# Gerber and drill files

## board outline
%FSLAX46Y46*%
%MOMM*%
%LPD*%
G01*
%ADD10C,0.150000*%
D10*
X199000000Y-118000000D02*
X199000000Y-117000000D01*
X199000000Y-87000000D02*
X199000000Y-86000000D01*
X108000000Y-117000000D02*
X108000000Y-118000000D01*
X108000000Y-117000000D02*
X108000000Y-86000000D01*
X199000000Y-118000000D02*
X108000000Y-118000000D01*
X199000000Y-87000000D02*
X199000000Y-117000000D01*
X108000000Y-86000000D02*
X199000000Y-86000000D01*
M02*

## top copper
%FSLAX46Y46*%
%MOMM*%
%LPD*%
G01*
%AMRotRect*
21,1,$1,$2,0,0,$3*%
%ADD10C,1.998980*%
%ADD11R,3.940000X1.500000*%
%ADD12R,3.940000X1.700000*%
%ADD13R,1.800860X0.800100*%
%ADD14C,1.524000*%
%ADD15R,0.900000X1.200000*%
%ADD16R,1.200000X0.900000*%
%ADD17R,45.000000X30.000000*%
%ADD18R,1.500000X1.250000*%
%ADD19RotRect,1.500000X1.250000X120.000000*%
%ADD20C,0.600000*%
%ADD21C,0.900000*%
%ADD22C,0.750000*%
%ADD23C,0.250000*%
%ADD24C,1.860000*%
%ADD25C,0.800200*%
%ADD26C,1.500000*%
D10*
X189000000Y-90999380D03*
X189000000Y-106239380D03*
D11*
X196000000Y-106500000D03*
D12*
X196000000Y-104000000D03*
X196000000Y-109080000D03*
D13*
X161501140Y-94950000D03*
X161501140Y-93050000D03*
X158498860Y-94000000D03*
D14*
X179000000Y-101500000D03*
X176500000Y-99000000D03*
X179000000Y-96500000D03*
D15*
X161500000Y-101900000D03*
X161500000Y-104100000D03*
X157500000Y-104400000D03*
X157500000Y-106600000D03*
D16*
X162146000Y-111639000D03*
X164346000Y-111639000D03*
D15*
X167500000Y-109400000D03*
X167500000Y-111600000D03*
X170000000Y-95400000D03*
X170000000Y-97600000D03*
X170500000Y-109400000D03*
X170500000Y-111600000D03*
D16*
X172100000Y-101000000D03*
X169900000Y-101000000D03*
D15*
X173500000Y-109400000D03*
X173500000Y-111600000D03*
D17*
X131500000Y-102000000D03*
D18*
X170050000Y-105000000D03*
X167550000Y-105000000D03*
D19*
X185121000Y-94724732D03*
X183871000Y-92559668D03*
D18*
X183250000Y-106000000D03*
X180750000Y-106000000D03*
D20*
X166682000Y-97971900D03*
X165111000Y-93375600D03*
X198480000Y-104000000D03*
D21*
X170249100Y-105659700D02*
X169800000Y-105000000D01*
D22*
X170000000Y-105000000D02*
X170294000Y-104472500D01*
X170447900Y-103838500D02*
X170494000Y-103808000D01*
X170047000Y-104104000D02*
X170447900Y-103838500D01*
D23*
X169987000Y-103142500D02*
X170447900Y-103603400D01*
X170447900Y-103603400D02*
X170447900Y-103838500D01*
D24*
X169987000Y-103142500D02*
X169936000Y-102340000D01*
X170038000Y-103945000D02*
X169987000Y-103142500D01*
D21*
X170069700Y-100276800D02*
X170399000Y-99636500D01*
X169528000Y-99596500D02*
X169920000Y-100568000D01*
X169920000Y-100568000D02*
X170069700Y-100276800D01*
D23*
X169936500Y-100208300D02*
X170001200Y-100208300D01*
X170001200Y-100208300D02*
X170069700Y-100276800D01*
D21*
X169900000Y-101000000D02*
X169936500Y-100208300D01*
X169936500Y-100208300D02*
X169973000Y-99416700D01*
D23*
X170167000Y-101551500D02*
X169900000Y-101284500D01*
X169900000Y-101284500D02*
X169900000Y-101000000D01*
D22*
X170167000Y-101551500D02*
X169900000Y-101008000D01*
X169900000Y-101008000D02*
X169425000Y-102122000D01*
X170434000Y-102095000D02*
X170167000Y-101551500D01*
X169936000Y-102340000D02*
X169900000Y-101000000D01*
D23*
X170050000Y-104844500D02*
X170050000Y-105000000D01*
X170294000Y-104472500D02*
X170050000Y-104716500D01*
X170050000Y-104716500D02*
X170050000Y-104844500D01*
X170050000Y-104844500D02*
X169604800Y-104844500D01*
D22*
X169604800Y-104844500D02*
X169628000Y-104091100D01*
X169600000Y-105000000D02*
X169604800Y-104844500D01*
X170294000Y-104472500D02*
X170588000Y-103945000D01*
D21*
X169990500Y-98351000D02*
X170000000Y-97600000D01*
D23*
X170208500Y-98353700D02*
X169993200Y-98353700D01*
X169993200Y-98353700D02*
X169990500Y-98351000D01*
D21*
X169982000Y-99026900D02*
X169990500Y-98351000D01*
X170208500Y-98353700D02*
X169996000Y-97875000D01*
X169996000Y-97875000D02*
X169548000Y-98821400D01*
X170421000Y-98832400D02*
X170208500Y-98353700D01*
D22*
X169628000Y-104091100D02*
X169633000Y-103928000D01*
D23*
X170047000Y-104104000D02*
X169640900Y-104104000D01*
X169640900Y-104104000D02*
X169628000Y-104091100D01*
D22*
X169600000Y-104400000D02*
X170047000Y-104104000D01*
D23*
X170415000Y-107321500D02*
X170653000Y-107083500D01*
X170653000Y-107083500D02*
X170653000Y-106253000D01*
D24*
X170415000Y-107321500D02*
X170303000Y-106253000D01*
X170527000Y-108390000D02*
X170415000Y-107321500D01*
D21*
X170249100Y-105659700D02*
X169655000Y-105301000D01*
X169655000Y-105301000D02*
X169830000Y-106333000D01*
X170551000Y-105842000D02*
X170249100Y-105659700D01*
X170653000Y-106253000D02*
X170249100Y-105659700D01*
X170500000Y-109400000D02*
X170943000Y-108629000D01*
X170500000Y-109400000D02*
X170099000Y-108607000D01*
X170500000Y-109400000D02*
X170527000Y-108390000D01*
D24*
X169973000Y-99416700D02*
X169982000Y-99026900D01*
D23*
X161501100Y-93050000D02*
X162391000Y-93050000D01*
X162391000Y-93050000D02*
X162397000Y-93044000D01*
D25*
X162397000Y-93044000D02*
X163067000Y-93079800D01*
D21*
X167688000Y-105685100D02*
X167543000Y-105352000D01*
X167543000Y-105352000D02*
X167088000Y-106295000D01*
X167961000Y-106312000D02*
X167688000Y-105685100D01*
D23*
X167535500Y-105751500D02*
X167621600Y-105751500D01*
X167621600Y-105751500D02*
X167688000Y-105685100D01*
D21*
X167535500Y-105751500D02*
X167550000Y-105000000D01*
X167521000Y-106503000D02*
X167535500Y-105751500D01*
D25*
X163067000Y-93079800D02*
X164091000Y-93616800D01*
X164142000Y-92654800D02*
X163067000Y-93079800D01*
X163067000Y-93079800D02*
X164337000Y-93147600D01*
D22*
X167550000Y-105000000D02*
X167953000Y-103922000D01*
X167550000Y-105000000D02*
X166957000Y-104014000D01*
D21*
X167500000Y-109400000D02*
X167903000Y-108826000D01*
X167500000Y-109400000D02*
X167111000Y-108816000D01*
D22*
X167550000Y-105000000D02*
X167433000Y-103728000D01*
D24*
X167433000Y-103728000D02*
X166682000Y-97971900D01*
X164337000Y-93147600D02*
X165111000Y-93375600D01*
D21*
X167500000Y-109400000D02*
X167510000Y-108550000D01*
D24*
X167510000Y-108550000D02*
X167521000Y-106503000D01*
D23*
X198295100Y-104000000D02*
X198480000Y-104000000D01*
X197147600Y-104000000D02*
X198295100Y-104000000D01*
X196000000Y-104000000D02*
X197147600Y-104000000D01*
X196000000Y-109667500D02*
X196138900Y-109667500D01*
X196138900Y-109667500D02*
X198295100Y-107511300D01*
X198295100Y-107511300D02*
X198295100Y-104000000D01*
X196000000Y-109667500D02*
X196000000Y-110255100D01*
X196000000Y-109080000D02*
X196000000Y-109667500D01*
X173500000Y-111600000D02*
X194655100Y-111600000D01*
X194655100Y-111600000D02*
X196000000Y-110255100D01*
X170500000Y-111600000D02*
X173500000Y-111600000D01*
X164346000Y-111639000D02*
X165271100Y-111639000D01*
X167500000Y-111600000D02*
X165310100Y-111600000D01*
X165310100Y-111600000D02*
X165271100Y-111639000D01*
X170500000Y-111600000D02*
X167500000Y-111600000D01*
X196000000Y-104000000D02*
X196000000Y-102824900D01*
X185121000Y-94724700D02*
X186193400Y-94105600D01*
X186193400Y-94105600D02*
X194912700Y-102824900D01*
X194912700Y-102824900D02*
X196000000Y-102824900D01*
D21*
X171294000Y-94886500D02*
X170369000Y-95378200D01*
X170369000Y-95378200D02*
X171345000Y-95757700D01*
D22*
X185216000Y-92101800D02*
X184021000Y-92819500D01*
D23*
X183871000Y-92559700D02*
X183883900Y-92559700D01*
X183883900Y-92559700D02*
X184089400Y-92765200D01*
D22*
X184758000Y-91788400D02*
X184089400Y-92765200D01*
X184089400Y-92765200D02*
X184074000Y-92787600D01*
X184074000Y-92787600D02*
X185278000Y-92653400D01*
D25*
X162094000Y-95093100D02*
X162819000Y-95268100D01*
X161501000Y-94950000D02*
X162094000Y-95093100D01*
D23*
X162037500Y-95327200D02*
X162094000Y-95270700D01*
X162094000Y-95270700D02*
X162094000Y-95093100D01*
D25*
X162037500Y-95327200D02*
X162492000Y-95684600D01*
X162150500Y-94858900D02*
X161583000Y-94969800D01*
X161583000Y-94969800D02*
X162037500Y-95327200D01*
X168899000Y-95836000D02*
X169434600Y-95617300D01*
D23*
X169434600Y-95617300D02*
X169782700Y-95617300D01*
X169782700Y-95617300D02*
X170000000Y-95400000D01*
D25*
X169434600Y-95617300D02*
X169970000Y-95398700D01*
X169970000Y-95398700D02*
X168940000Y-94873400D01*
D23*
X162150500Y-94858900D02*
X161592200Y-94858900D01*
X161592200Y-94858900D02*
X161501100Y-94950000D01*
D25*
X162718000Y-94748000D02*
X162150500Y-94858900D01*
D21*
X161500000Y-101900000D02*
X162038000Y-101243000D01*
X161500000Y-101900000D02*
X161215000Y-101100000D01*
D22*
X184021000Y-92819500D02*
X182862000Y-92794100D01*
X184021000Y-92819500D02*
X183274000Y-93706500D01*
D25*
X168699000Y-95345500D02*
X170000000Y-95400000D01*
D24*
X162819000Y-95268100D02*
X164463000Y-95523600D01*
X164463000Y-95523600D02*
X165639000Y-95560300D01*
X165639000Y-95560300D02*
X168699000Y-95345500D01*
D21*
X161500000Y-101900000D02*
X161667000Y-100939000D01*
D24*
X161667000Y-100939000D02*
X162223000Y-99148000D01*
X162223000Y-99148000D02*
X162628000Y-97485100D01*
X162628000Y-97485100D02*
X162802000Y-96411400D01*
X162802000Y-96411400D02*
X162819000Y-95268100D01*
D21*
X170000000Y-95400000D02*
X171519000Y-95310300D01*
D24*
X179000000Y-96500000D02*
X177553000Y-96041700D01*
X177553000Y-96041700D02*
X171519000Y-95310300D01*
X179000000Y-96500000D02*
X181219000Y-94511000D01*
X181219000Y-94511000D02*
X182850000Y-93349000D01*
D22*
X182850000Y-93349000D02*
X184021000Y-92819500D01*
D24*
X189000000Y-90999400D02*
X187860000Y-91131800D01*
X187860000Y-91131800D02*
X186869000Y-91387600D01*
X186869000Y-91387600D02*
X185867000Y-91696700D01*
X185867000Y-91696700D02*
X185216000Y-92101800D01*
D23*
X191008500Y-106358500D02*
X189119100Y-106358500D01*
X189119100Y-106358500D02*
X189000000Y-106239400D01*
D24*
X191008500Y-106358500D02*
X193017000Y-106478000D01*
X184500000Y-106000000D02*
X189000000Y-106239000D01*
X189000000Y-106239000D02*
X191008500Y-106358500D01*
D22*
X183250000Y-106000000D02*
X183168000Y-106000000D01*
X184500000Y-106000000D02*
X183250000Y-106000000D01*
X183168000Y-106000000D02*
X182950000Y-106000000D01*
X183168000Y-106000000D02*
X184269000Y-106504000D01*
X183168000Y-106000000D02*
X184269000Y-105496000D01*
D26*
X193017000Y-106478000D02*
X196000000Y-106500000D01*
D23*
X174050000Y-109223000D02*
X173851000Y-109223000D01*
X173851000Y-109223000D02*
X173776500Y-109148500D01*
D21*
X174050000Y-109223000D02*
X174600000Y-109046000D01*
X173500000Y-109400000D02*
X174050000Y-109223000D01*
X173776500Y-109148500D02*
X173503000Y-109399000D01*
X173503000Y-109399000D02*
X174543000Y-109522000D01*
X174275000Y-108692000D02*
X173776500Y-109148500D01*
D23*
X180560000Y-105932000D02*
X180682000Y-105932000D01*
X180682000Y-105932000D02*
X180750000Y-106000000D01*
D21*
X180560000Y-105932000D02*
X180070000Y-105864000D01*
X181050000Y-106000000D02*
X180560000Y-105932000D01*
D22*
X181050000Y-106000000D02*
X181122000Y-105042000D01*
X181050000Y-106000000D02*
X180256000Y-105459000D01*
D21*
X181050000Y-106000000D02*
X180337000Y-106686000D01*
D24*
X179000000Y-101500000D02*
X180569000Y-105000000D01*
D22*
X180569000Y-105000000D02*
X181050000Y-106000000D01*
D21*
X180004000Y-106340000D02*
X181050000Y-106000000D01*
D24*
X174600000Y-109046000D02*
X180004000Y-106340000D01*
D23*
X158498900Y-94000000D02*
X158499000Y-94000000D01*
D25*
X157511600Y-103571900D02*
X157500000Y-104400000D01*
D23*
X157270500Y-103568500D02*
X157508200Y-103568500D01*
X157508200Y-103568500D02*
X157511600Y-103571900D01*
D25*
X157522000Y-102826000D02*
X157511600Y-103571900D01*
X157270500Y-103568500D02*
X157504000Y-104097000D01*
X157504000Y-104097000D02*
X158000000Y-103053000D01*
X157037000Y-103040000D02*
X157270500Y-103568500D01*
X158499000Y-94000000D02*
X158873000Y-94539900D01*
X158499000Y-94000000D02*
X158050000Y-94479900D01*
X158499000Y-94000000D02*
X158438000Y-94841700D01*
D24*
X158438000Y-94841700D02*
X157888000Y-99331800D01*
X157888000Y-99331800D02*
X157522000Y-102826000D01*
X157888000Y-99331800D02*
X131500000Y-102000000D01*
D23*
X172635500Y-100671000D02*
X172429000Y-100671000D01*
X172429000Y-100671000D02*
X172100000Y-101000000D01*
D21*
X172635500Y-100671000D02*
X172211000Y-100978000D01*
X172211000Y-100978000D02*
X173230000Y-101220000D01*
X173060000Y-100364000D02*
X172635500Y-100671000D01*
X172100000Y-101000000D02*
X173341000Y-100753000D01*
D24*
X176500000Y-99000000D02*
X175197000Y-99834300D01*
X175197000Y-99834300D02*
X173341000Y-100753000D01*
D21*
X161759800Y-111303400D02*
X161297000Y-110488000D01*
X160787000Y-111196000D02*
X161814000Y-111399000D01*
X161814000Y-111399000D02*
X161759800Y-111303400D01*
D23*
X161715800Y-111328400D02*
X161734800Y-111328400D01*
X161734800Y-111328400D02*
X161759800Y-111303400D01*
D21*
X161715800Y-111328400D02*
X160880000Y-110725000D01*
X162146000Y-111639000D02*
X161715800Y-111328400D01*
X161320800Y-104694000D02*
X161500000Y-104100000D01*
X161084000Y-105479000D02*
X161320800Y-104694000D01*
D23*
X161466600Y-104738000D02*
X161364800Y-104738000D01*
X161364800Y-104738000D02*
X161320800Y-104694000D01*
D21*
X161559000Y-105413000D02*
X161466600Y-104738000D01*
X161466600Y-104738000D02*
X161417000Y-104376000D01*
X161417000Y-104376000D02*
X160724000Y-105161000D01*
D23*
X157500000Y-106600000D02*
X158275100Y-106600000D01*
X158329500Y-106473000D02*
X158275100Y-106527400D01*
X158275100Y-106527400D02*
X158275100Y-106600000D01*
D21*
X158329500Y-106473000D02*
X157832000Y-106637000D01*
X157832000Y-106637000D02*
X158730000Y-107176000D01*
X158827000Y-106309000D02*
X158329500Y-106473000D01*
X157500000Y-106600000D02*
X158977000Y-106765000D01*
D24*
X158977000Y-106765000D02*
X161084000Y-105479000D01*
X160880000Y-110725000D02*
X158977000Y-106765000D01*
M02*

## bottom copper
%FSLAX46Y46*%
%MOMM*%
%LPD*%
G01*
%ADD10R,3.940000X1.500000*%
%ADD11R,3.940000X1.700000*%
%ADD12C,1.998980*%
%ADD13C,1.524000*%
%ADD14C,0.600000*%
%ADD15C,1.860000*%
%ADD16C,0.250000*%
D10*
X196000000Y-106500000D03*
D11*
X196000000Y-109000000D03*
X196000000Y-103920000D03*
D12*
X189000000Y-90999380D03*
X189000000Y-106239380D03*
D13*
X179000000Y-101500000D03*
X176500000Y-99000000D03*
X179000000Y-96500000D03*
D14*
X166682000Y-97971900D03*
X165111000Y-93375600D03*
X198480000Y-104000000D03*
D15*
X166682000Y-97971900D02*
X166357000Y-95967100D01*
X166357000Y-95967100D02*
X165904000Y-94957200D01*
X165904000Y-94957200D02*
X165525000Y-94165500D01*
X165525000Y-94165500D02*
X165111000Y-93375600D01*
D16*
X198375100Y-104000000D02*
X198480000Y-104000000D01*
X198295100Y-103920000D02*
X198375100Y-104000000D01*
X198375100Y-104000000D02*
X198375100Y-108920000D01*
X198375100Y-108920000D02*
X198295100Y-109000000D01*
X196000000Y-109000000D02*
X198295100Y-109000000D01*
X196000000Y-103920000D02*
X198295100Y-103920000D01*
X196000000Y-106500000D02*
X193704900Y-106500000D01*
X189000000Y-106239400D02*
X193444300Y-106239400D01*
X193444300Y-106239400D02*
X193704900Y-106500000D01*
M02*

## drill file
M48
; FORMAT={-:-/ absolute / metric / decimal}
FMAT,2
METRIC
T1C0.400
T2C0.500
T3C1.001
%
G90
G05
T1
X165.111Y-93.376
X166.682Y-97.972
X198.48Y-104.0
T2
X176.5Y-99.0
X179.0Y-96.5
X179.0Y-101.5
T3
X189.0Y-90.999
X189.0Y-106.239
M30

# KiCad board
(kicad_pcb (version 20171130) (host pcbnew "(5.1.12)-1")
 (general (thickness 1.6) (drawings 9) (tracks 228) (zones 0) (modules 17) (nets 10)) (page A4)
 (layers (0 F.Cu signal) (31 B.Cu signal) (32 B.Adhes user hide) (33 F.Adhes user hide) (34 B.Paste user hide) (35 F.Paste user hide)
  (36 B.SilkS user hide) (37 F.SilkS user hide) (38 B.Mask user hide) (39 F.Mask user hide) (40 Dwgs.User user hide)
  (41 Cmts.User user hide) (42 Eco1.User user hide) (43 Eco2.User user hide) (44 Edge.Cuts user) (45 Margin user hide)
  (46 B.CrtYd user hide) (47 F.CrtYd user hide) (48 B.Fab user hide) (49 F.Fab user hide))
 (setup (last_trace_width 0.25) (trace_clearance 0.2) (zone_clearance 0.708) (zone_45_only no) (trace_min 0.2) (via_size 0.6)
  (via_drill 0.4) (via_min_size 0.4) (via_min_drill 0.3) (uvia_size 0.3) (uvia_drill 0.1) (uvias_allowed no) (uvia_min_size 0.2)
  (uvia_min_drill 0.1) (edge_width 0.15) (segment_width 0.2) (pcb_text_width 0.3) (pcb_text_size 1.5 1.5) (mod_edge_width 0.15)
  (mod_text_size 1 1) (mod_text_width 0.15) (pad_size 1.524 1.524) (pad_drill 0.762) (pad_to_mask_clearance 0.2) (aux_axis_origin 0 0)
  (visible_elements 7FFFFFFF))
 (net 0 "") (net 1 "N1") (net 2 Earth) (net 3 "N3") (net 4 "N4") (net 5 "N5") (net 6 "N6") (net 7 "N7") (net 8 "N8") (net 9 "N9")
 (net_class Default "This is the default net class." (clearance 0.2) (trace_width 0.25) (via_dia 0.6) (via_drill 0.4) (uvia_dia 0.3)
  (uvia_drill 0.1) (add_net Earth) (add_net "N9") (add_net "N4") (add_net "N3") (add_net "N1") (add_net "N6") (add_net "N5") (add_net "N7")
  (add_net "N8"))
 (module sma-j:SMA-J (layer B.Cu) (at 196 109)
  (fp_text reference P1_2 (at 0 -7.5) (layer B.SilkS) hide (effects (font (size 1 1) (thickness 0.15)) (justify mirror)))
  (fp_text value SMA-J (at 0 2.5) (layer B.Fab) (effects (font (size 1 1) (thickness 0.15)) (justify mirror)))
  (pad 1 smd rect (at 0 -2.5) (size 3.94 1.5) (layers B.Cu B.Paste B.Mask) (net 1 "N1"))
  (pad 2 smd rect (at 0 0) (size 3.94 1.7) (layers B.Cu B.Paste B.Mask) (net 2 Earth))
  (pad 2 smd rect (at 0 -5.08) (size 3.94 1.7) (layers B.Cu B.Paste B.Mask) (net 2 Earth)))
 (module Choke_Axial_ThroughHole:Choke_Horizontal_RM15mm (layer F.Cu) (at 189 98.5 270)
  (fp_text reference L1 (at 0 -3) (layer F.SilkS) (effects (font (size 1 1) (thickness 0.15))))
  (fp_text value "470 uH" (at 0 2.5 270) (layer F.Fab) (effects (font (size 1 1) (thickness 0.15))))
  (pad 1 thru_hole circle (at -7.50062 0 270) (size 1.99898 1.99898) (drill 1.00076) (layers *.Cu *.Mask F.SilkS) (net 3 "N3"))
  (pad 2 thru_hole circle (at 7.73938 0 270) (size 1.99898 1.99898) (drill 1.00076) (layers *.Cu *.Mask F.SilkS) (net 1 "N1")))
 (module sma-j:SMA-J (layer F.Cu) (at 196 104)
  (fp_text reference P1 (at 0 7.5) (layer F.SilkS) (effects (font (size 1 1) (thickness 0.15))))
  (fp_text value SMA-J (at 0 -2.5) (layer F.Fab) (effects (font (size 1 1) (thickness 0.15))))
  (pad 1 smd rect (at 0 2.5) (size 3.94 1.5) (layers F.Cu F.Paste F.Mask) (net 1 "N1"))
  (pad 2 smd rect (at 0 0) (size 3.94 1.7) (layers F.Cu F.Paste F.Mask) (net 2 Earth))
  (pad 2 smd rect (at 0 5.08) (size 3.94 1.7) (layers F.Cu F.Paste F.Mask) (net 2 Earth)))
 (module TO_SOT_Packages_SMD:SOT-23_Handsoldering (layer F.Cu) (at 160 94 90)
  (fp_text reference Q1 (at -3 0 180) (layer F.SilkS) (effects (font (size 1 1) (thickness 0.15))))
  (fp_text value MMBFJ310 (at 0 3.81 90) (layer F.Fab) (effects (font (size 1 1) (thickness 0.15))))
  (pad 1 smd rect (at -0.95 1.50114 90) (size 0.8001 1.80086) (layers F.Cu F.Paste F.Mask) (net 3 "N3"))
  (pad 2 smd rect (at 0.95 1.50114 90) (size 0.8001 1.80086) (layers F.Cu F.Paste F.Mask) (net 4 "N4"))
  (pad 3 smd rect (at 0 -1.50114 90) (size 0.8001 1.80086) (layers F.Cu F.Paste F.Mask) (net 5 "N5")))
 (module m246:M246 (layer F.Cu) (at 179 99 270)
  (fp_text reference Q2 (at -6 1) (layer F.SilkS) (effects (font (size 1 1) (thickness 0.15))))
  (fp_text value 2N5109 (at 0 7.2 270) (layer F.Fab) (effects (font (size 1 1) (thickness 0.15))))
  (pad 1 thru_hole circle (at 2.5 0 270) (size 1.524 1.524) (drill 0.5) (layers *.Cu *.Mask F.SilkS) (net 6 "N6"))
  (pad 2 thru_hole circle (at 0 2.5 270) (size 1.524 1.524) (drill 0.5) (layers *.Cu *.Mask F.SilkS) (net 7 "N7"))
  (pad 3 thru_hole circle (at -2.5 0 270) (size 1.524 1.524) (drill 0.5) (layers *.Cu *.Mask F.SilkS) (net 3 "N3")))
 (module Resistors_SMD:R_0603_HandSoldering (layer F.Cu) (at 161.5 103 270)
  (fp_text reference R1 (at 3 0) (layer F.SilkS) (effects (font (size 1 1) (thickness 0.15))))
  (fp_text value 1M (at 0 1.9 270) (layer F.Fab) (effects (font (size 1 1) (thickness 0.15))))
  (pad 1 smd rect (at -1.1 0 270) (size 1.2 0.9) (layers F.Cu F.Paste F.Mask) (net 3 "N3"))
  (pad 2 smd rect (at 1.1 0 270) (size 1.2 0.9) (layers F.Cu F.Paste F.Mask) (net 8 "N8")))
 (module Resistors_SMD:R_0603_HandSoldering (layer F.Cu) (at 157.5 105.5 270)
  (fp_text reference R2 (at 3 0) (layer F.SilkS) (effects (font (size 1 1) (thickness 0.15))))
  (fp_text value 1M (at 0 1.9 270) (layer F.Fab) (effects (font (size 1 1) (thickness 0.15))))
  (pad 1 smd rect (at -1.1 0 270) (size 1.2 0.9) (layers F.Cu F.Paste F.Mask) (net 5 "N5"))
  (pad 2 smd rect (at 1.1 0 270) (size 1.2 0.9) (layers F.Cu F.Paste F.Mask) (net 8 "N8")))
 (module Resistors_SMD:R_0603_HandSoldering (layer F.Cu) (at 163.246 111.639)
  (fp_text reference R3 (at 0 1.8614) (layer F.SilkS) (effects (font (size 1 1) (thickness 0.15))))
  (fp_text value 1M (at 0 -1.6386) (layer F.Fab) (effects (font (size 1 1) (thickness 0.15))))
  (pad 1 smd rect (at -1.1 0) (size 1.2 0.9) (layers F.Cu F.Paste F.Mask) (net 8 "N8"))
  (pad 2 smd rect (at 1.1 0) (size 1.2 0.9) (layers F.Cu F.Paste F.Mask) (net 2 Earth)))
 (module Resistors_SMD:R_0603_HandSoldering (layer F.Cu) (at 167.5 110.5 270)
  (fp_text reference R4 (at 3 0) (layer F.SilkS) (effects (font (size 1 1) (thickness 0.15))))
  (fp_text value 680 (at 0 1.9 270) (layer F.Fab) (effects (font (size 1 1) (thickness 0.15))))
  (pad 1 smd rect (at -1.1 0 270) (size 1.2 0.9) (layers F.Cu F.Paste F.Mask) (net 4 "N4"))
  (pad 2 smd rect (at 1.1 0 270) (size 1.2 0.9) (layers F.Cu F.Paste F.Mask) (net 2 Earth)))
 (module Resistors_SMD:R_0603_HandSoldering (layer F.Cu) (at 170 96.5 270)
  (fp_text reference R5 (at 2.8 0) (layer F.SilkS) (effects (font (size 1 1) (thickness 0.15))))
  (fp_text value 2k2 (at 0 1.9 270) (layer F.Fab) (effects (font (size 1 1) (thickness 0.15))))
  (pad 1 smd rect (at -1.1 0 270) (size 1.2 0.9) (layers F.Cu F.Paste F.Mask) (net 3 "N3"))
  (pad 2 smd rect (at 1.1 0 270) (size 1.2 0.9) (layers F.Cu F.Paste F.Mask) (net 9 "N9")))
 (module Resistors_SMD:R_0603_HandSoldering (layer F.Cu) (at 170.5 110.5 270)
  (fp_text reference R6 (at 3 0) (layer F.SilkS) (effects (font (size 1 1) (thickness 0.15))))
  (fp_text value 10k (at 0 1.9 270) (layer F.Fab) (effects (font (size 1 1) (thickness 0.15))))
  (pad 1 smd rect (at -1.1 0 270) (size 1.2 0.9) (layers F.Cu F.Paste F.Mask) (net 9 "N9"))
  (pad 2 smd rect (at 1.1 0 270) (size 1.2 0.9) (layers F.Cu F.Paste F.Mask) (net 2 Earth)))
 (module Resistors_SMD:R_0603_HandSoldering (layer F.Cu) (at 171 101 180)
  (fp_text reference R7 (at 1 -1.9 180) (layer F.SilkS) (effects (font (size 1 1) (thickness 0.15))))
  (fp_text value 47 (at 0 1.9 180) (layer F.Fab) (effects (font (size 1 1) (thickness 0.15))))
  (pad 1 smd rect (at -1.1 0 180) (size 1.2 0.9) (layers F.Cu F.Paste F.Mask) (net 7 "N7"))
  (pad 2 smd rect (at 1.1 0 180) (size 1.2 0.9) (layers F.Cu F.Paste F.Mask) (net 9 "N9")))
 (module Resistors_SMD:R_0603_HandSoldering (layer F.Cu) (at 173.5 110.5 270)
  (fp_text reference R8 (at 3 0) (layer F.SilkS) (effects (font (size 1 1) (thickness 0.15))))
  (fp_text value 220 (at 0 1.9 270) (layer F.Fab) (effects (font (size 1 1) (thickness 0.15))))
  (pad 1 smd rect (at -1.1 0 270) (size 1.2 0.9) (layers F.Cu F.Paste F.Mask) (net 6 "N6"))
  (pad 2 smd rect (at 1.1 0 270) (size 1.2 0.9) (layers F.Cu F.Paste F.Mask) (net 2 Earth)))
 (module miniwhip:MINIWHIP (layer F.Cu) (at 109 87)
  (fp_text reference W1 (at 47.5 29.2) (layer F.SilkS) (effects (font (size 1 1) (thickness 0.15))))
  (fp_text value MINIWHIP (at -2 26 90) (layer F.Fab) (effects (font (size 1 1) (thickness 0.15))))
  (pad 1 smd rect (at 22.5 15) (size 45 30) (layers F.Cu F.Paste F.Mask) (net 5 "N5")))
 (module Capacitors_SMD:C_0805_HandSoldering (layer F.Cu) (at 168.8 105 180)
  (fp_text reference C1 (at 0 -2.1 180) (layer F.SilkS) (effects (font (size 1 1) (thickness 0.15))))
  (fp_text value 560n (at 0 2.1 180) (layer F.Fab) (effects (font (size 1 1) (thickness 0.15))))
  (pad 1 smd rect (at -1.25 0 180) (size 1.5 1.25) (layers F.Cu F.Paste F.Mask) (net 9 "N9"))
  (pad 2 smd rect (at 1.25 0 180) (size 1.5 1.25) (layers F.Cu F.Paste F.Mask) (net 4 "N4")))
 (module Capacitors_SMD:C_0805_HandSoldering (layer F.Cu) (at 184.496 93.6422 120)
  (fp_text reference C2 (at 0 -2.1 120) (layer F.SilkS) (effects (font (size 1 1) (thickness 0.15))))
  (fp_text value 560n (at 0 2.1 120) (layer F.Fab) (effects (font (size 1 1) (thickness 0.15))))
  (pad 1 smd rect (at -1.25 0 120) (size 1.5 1.25) (layers F.Cu F.Paste F.Mask) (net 2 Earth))
  (pad 2 smd rect (at 1.25 0 120) (size 1.5 1.25) (layers F.Cu F.Paste F.Mask) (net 3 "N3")))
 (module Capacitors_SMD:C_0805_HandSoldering (layer F.Cu) (at 182 106 180)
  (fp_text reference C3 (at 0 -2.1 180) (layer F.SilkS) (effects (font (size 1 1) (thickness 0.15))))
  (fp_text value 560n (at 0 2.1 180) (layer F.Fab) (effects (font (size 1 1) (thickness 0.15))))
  (pad 1 smd rect (at -1.25 0 180) (size 1.5 1.25) (layers F.Cu F.Paste F.Mask) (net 1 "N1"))
  (pad 2 smd rect (at 1.25 0 180) (size 1.5 1.25) (layers F.Cu F.Paste F.Mask) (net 6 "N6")))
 (gr_line (start 199 118) (end 199 117) (layer Edge.Cuts) (width 0.15))
 (gr_line (start 199 87) (end 199 86) (layer Edge.Cuts) (width 0.15))
 (gr_line (start 108 117) (end 108 118) (layer Edge.Cuts) (width 0.15))
 (gr_line (start 108 117) (end 108 86) (layer Edge.Cuts) (width 0.15))
 (gr_line (start 199 118) (end 108 118) (layer Edge.Cuts) (width 0.15))
 (gr_line (start 199 87) (end 199 117) (layer Edge.Cuts) (width 0.15))
 (gr_line (start 108 86) (end 199 86) (layer Edge.Cuts) (width 0.15))
 (segment (start 170.2491 105.6597) (end 169.8 105) (width 0.9) (layer F.Cu) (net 9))
 (segment (start 170 105) (end 170.294 104.4725) (width 0.75) (layer F.Cu) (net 9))
 (segment (start 170.4479 103.8385) (end 170.494 103.808) (width 0.75) (layer F.Cu) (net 9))
 (segment (start 170.047 104.104) (end 170.4479 103.8385) (width 0.75) (layer F.Cu) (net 9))
 (segment (start 169.987 103.1425) (end 170.4479 103.6034) (width 0.25) (layer F.Cu) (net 9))
 (segment (start 170.4479 103.6034) (end 170.4479 103.8385) (width 0.25) (layer F.Cu) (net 9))
 (segment (start 169.987 103.1425) (end 169.936 102.34) (width 1.86) (layer F.Cu) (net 9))
 (segment (start 170.038 103.945) (end 169.987 103.1425) (width 1.86) (layer F.Cu) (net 9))
 (segment (start 170.0697 100.2768) (end 170.399 99.6365) (width 0.9) (layer F.Cu) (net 9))
 (segment (start 169.528 99.5965) (end 169.92 100.568) (width 0.9) (layer F.Cu) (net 9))
 (segment (start 169.92 100.568) (end 170.0697 100.2768) (width 0.9) (layer F.Cu) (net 9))
 (segment (start 169.9365 100.2083) (end 170.0012 100.2083) (width 0.25) (layer F.Cu) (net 9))
 (segment (start 170.0012 100.2083) (end 170.0697 100.2768) (width 0.25) (layer F.Cu) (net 9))
 (segment (start 169.9 101) (end 169.9365 100.2083) (width 0.9) (layer F.Cu) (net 9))
 (segment (start 169.9365 100.2083) (end 169.973 99.4167) (width 0.9) (layer F.Cu) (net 9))
 (segment (start 170.167 101.5515) (end 169.9 101.2845) (width 0.25) (layer F.Cu) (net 9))
 (segment (start 169.9 101.2845) (end 169.9 101) (width 0.25) (layer F.Cu) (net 9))
 (segment (start 170.167 101.5515) (end 169.9 101.008) (width 0.75) (layer F.Cu) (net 9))
 (segment (start 169.9 101.008) (end 169.425 102.122) (width 0.75) (layer F.Cu) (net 9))
 (segment (start 170.434 102.095) (end 170.167 101.5515) (width 0.75) (layer F.Cu) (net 9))
 (segment (start 169.936 102.34) (end 169.9 101) (width 0.75) (layer F.Cu) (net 9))
 (segment (start 170.05 104.8445) (end 170.05 105) (width 0.25) (layer F.Cu) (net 9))
 (segment (start 170.294 104.4725) (end 170.05 104.7165) (width 0.25) (layer F.Cu) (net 9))
 (segment (start 170.05 104.7165) (end 170.05 104.8445) (width 0.25) (layer F.Cu) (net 9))
 (segment (start 170.05 104.8445) (end 169.6048 104.8445) (width 0.25) (layer F.Cu) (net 9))
 (segment (start 169.6048 104.8445) (end 169.628 104.0911) (width 0.75) (layer F.Cu) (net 9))
 (segment (start 169.6 105) (end 169.6048 104.8445) (width 0.75) (layer F.Cu) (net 9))
 (segment (start 170.294 104.4725) (end 170.588 103.945) (width 0.75) (layer F.Cu) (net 9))
 (segment (start 169.9905 98.351) (end 170 97.6) (width 0.9) (layer F.Cu) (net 9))
 (segment (start 170.2085 98.3537) (end 169.9932 98.3537) (width 0.25) (layer F.Cu) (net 9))
 (segment (start 169.9932 98.3537) (end 169.9905 98.351) (width 0.25) (layer F.Cu) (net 9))
 (segment (start 169.982 99.0269) (end 169.9905 98.351) (width 0.9) (layer F.Cu) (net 9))
 (segment (start 170.2085 98.3537) (end 169.996 97.875) (width 0.9) (layer F.Cu) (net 9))
 (segment (start 169.996 97.875) (end 169.548 98.8214) (width 0.9) (layer F.Cu) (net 9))
 (segment (start 170.421 98.8324) (end 170.2085 98.3537) (width 0.9) (layer F.Cu) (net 9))
 (segment (start 169.628 104.0911) (end 169.633 103.928) (width 0.75) (layer F.Cu) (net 9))
 (segment (start 170.047 104.104) (end 169.6409 104.104) (width 0.25) (layer F.Cu) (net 9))
 (segment (start 169.6409 104.104) (end 169.628 104.0911) (width 0.25) (layer F.Cu) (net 9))
 (segment (start 169.6 104.4) (end 170.047 104.104) (width 0.75) (layer F.Cu) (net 9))
 (segment (start 170.415 107.3215) (end 170.653 107.0835) (width 0.25) (layer F.Cu) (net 9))
 (segment (start 170.653 107.0835) (end 170.653 106.253) (width 0.25) (layer F.Cu) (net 9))
 (segment (start 170.415 107.3215) (end 170.303 106.253) (width 1.86) (layer F.Cu) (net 9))
 (segment (start 170.527 108.39) (end 170.415 107.3215) (width 1.86) (layer F.Cu) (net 9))
 (segment (start 170.2491 105.6597) (end 169.655 105.301) (width 0.9) (layer F.Cu) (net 9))
 (segment (start 169.655 105.301) (end 169.83 106.333) (width 0.9) (layer F.Cu) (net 9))
 (segment (start 170.551 105.842) (end 170.2491 105.6597) (width 0.9) (layer F.Cu) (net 9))
 (segment (start 170.653 106.253) (end 170.2491 105.6597) (width 0.9) (layer F.Cu) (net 9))
 (segment (start 170.5 109.4) (end 170.943 108.629) (width 0.9) (layer F.Cu) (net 9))
 (segment (start 170.5 109.4) (end 170.099 108.607) (width 0.9) (layer F.Cu) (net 9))
 (segment (start 170.5 109.4) (end 170.527 108.39) (width 0.9) (layer F.Cu) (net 9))
 (segment (start 169.973 99.4167) (end 169.982 99.0269) (width 1.86) (layer F.Cu) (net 9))
 (segment (start 161.5011 93.05) (end 162.391 93.05) (width 0.25) (layer F.Cu) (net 4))
 (segment (start 162.391 93.05) (end 162.397 93.044) (width 0.25) (layer F.Cu) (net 4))
 (segment (start 162.397 93.044) (end 163.067 93.0798) (width 0.8002) (layer F.Cu) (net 4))
 (segment (start 167.688 105.6851) (end 167.543 105.352) (width 0.9) (layer F.Cu) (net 4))
 (segment (start 167.543 105.352) (end 167.088 106.295) (width 0.9) (layer F.Cu) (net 4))
 (segment (start 167.961 106.312) (end 167.688 105.6851) (width 0.9) (layer F.Cu) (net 4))
 (segment (start 167.5355 105.7515) (end 167.6216 105.7515) (width 0.25) (layer F.Cu) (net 4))
 (segment (start 167.6216 105.7515) (end 167.688 105.6851) (width 0.25) (layer F.Cu) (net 4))
 (segment (start 167.5355 105.7515) (end 167.55 105) (width 0.9) (layer F.Cu) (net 4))
 (segment (start 167.521 106.503) (end 167.5355 105.7515) (width 0.9) (layer F.Cu) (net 4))
 (segment (start 163.067 93.0798) (end 164.091 93.6168) (width 0.8002) (layer F.Cu) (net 4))
 (segment (start 164.142 92.6548) (end 163.067 93.0798) (width 0.8002) (layer F.Cu) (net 4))
 (segment (start 163.067 93.0798) (end 164.337 93.1476) (width 0.8002) (layer F.Cu) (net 4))
 (segment (start 167.55 105) (end 167.953 103.922) (width 0.75) (layer F.Cu) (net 4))
 (segment (start 167.55 105) (end 166.957 104.014) (width 0.75) (layer F.Cu) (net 4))
 (segment (start 167.5 109.4) (end 167.903 108.826) (width 0.9) (layer F.Cu) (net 4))
 (segment (start 167.5 109.4) (end 167.111 108.816) (width 0.9) (layer F.Cu) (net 4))
 (segment (start 167.55 105) (end 167.433 103.728) (width 0.75) (layer F.Cu) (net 4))
 (segment (start 167.433 103.728) (end 166.682 97.9719) (width 1.86) (layer F.Cu) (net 4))
 (segment (start 164.337 93.1476) (end 165.111 93.3756) (width 1.86) (layer F.Cu) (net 4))
 (segment (start 167.5 109.4) (end 167.51 108.55) (width 0.9) (layer F.Cu) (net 4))
 (segment (start 167.51 108.55) (end 167.521 106.503) (width 1.86) (layer F.Cu) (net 4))
 (segment (start 166.682 97.9719) (end 166.357 95.9671) (width 1.86) (layer B.Cu) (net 4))
 (segment (start 166.357 95.9671) (end 165.904 94.9572) (width 1.86) (layer B.Cu) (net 4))
 (segment (start 165.904 94.9572) (end 165.525 94.1655) (width 1.86) (layer B.Cu) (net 4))
 (segment (start 165.525 94.1655) (end 165.111 93.3756) (width 1.86) (layer B.Cu) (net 4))
 (via (at 166.682 97.9719) (size 0.6) (layers F.Cu B.Cu) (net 4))
 (via (at 165.111 93.3756) (size 0.6) (layers F.Cu B.Cu) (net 4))
 (segment (start 198.3751 104) (end 198.48 104) (width 0.25) (layer B.Cu) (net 2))
 (segment (start 198.2951 103.92) (end 198.3751 104) (width 0.25) (layer B.Cu) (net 2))
 (segment (start 198.3751 104) (end 198.3751 108.92) (width 0.25) (layer B.Cu) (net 2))
 (segment (start 198.3751 108.92) (end 198.2951 109) (width 0.25) (layer B.Cu) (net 2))
 (segment (start 196 109) (end 198.2951 109) (width 0.25) (layer B.Cu) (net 2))
 (segment (start 196 103.92) (end 198.2951 103.92) (width 0.25) (layer B.Cu) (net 2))
 (segment (start 198.2951 104) (end 198.48 104) (width 0.25) (layer F.Cu) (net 2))
 (segment (start 197.1476 104) (end 198.2951 104) (width 0.25) (layer F.Cu) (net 2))
 (segment (start 196 104) (end 197.1476 104) (width 0.25) (layer F.Cu) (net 2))
 (segment (start 196 109.6675) (end 196.1389 109.6675) (width 0.25) (layer F.Cu) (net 2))
 (segment (start 196.1389 109.6675) (end 198.2951 107.5113) (width 0.25) (layer F.Cu) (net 2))
 (segment (start 198.2951 107.5113) (end 198.2951 104) (width 0.25) (layer F.Cu) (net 2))
 (segment (start 196 109.6675) (end 196 110.2551) (width 0.25) (layer F.Cu) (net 2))
 (segment (start 196 109.08) (end 196 109.6675) (width 0.25) (layer F.Cu) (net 2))
 (segment (start 173.5 111.6) (end 194.6551 111.6) (width 0.25) (layer F.Cu) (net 2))
 (segment (start 194.6551 111.6) (end 196 110.2551) (width 0.25) (layer F.Cu) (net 2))
 (segment (start 170.5 111.6) (end 173.5 111.6) (width 0.25) (layer F.Cu) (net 2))
 (segment (start 164.346 111.639) (end 165.2711 111.639) (width 0.25) (layer F.Cu) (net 2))
 (segment (start 167.5 111.6) (end 165.3101 111.6) (width 0.25) (layer F.Cu) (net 2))
 (segment (start 165.3101 111.6) (end 165.2711 111.639) (width 0.25) (layer F.Cu) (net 2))
 (segment (start 170.5 111.6) (end 167.5 111.6) (width 0.25) (layer F.Cu) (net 2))
 (segment (start 196 104) (end 196 102.8249) (width 0.25) (layer F.Cu) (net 2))
 (segment (start 185.121 94.7247) (end 186.1934 94.1056) (width 0.25) (layer F.Cu) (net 2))
 (segment (start 186.1934 94.1056) (end 194.9127 102.8249) (width 0.25) (layer F.Cu) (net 2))
 (segment (start 194.9127 102.8249) (end 196 102.8249) (width 0.25) (layer F.Cu) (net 2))
 (via (at 198.48 104) (size 0.6) (layers F.Cu B.Cu) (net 2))
 (segment (start 171.294 94.8865) (end 170.369 95.3782) (width 0.9) (layer F.Cu) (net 3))
 (segment (start 170.369 95.3782) (end 171.345 95.7577) (width 0.9) (layer F.Cu) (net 3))
 (segment (start 185.216 92.1018) (end 184.021 92.8195) (width 0.75) (layer F.Cu) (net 3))
 (segment (start 183.871 92.5597) (end 183.8839 92.5597) (width 0.25) (layer F.Cu) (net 3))
 (segment (start 183.8839 92.5597) (end 184.0894 92.7652) (width 0.25) (layer F.Cu) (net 3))
 (segment (start 184.758 91.7884) (end 184.0894 92.7652) (width 0.75) (layer F.Cu) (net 3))
 (segment (start 184.0894 92.7652) (end 184.074 92.7876) (width 0.75) (layer F.Cu) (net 3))
 (segment (start 184.074 92.7876) (end 185.278 92.6534) (width 0.75) (layer F.Cu) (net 3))
 (segment (start 162.094 95.0931) (end 162.819 95.2681) (width 0.8002) (layer F.Cu) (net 3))
 (segment (start 161.501 94.95) (end 162.094 95.0931) (width 0.8002) (layer F.Cu) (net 3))
 (segment (start 162.0375 95.3272) (end 162.094 95.2707) (width 0.25) (layer F.Cu) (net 3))
 (segment (start 162.094 95.2707) (end 162.094 95.0931) (width 0.25) (layer F.Cu) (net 3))
 (segment (start 162.0375 95.3272) (end 162.492 95.6846) (width 0.8002) (layer F.Cu) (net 3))
 (segment (start 162.1505 94.8589) (end 161.583 94.9698) (width 0.8002) (layer F.Cu) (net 3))
 (segment (start 161.583 94.9698) (end 162.0375 95.3272) (width 0.8002) (layer F.Cu) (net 3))
 (segment (start 168.899 95.836) (end 169.4346 95.6173) (width 0.8002) (layer F.Cu) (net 3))
 (segment (start 169.4346 95.6173) (end 169.7827 95.6173) (width 0.25) (layer F.Cu) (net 3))
 (segment (start 169.7827 95.6173) (end 170 95.4) (width 0.25) (layer F.Cu) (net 3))
 (segment (start 169.4346 95.6173) (end 169.97 95.3987) (width 0.8002) (layer F.Cu) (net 3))
 (segment (start 169.97 95.3987) (end 168.94 94.8734) (width 0.8002) (layer F.Cu) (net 3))
 (segment (start 162.1505 94.8589) (end 161.5922 94.8589) (width 0.25) (layer F.Cu) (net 3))
 (segment (start 161.5922 94.8589) (end 161.5011 94.95) (width 0.25) (layer F.Cu) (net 3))
 (segment (start 162.718 94.748) (end 162.1505 94.8589) (width 0.8002) (layer F.Cu) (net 3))
 (segment (start 161.5 101.9) (end 162.038 101.243) (width 0.9) (layer F.Cu) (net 3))
 (segment (start 161.5 101.9) (end 161.215 101.1) (width 0.9) (layer F.Cu) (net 3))
 (segment (start 184.021 92.8195) (end 182.862 92.7941) (width 0.75) (layer F.Cu) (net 3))
 (segment (start 184.021 92.8195) (end 183.274 93.7065) (width 0.75) (layer F.Cu) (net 3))
 (segment (start 168.699 95.3455) (end 170 95.4) (width 0.8002) (layer F.Cu) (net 3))
 (segment (start 162.819 95.2681) (end 164.463 95.5236) (width 1.86) (layer F.Cu) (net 3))
 (segment (start 164.463 95.5236) (end 165.639 95.5603) (width 1.86) (layer F.Cu) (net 3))
 (segment (start 165.639 95.5603) (end 168.699 95.3455) (width 1.86) (layer F.Cu) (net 3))
 (segment (start 161.5 101.9) (end 161.667 100.939) (width 0.9) (layer F.Cu) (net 3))
 (segment (start 161.667 100.939) (end 162.223 99.148) (width 1.86) (layer F.Cu) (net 3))
 (segment (start 162.223 99.148) (end 162.628 97.4851) (width 1.86) (layer F.Cu) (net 3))
 (segment (start 162.628 97.4851) (end 162.802 96.4114) (width 1.86) (layer F.Cu) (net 3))
 (segment (start 162.802 96.4114) (end 162.819 95.2681) (width 1.86) (layer F.Cu) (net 3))
 (segment (start 170 95.4) (end 171.519 95.3103) (width 0.9) (layer F.Cu) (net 3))
 (segment (start 179 96.5) (end 177.553 96.0417) (width 1.86) (layer F.Cu) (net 3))
 (segment (start 177.553 96.0417) (end 171.519 95.3103) (width 1.86) (layer F.Cu) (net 3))
 (segment (start 179 96.5) (end 181.219 94.511) (width 1.86) (layer F.Cu) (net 3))
 (segment (start 181.219 94.511) (end 182.85 93.349) (width 1.86) (layer F.Cu) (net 3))
 (segment (start 182.85 93.349) (end 184.021 92.8195) (width 0.75) (layer F.Cu) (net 3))
 (segment (start 189 90.9994) (end 187.86 91.1318) (width 1.86) (layer F.Cu) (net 3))
 (segment (start 187.86 91.1318) (end 186.869 91.3876) (width 1.86) (layer F.Cu) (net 3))
 (segment (start 186.869 91.3876) (end 185.867 91.6967) (width 1.86) (layer F.Cu) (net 3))
 (segment (start 185.867 91.6967) (end 185.216 92.1018) (width 1.86) (layer F.Cu) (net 3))
 (segment (start 196 106.5) (end 193.7049 106.5) (width 0.25) (layer B.Cu) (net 1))
 (segment (start 189 106.2394) (end 193.4443 106.2394) (width 0.25) (layer B.Cu) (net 1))
 (segment (start 193.4443 106.2394) (end 193.7049 106.5) (width 0.25) (layer B.Cu) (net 1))
 (segment (start 191.0085 106.3585) (end 189.1191 106.3585) (width 0.25) (layer F.Cu) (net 1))
 (segment (start 189.1191 106.3585) (end 189 106.2394) (width 0.25) (layer F.Cu) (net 1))
 (segment (start 191.0085 106.3585) (end 193.017 106.478) (width 1.86) (layer F.Cu) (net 1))
 (segment (start 184.5 106) (end 189 106.239) (width 1.86) (layer F.Cu) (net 1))
 (segment (start 189 106.239) (end 191.0085 106.3585) (width 1.86) (layer F.Cu) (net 1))
 (segment (start 183.25 106) (end 183.168 106) (width 0.75) (layer F.Cu) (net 1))
 (segment (start 184.5 106) (end 183.25 106) (width 0.75) (layer F.Cu) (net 1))
 (segment (start 183.168 106) (end 182.95 106) (width 0.75) (layer F.Cu) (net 1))
 (segment (start 183.168 106) (end 184.269 106.504) (width 0.75) (layer F.Cu) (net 1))
 (segment (start 183.168 106) (end 184.269 105.496) (width 0.75) (layer F.Cu) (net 1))
 (segment (start 193.017 106.478) (end 196 106.5) (width 1.5) (layer F.Cu) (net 1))
 (segment (start 174.05 109.223) (end 173.851 109.223) (width 0.25) (layer F.Cu) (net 6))
 (segment (start 173.851 109.223) (end 173.7765 109.1485) (width 0.25) (layer F.Cu) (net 6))
 (segment (start 174.05 109.223) (end 174.6 109.046) (width 0.9) (layer F.Cu) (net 6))
 (segment (start 173.5 109.4) (end 174.05 109.223) (width 0.9) (layer F.Cu) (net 6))
 (segment (start 173.7765 109.1485) (end 173.503 109.399) (width 0.9) (layer F.Cu) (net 6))
 (segment (start 173.503 109.399) (end 174.543 109.522) (width 0.9) (layer F.Cu) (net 6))
 (segment (start 174.275 108.692) (end 173.7765 109.1485) (width 0.9) (layer F.Cu) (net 6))
 (segment (start 180.56 105.932) (end 180.682 105.932) (width 0.25) (layer F.Cu) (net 6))
 (segment (start 180.682 105.932) (end 180.75 106) (width 0.25) (layer F.Cu) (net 6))
 (segment (start 180.56 105.932) (end 180.07 105.864) (width 0.9) (layer F.Cu) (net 6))
 (segment (start 181.05 106) (end 180.56 105.932) (width 0.9) (layer F.Cu) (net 6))
 (segment (start 181.05 106) (end 181.122 105.042) (width 0.75) (layer F.Cu) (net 6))
 (segment (start 181.05 106) (end 180.256 105.459) (width 0.75) (layer F.Cu) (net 6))
 (segment (start 181.05 106) (end 180.337 106.686) (width 0.9) (layer F.Cu) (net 6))
 (segment (start 179 101.5) (end 180.569 105) (width 1.86) (layer F.Cu) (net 6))
 (segment (start 180.569 105) (end 181.05 106) (width 0.75) (layer F.Cu) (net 6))
 (segment (start 180.004 106.34) (end 181.05 106) (width 0.9) (layer F.Cu) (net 6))
 (segment (start 174.6 109.046) (end 180.004 106.34) (width 1.86) (layer F.Cu) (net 6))
 (segment (start 158.4989 94) (end 158.499 94) (width 0.25) (layer F.Cu) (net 5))
 (segment (start 157.5116 103.5719) (end 157.5 104.4) (width 0.8002) (layer F.Cu) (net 5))
 (segment (start 157.2705 103.5685) (end 157.5082 103.5685) (width 0.25) (layer F.Cu) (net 5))
 (segment (start 157.5082 103.5685) (end 157.5116 103.5719) (width 0.25) (layer F.Cu) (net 5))
 (segment (start 157.522 102.826) (end 157.5116 103.5719) (width 0.8002) (layer F.Cu) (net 5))
 (segment (start 157.2705 103.5685) (end 157.504 104.097) (width 0.8002) (layer F.Cu) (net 5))
 (segment (start 157.504 104.097) (end 158 103.053) (width 0.8002) (layer F.Cu) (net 5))
 (segment (start 157.037 103.04) (end 157.2705 103.5685) (width 0.8002) (layer F.Cu) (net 5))
 (segment (start 158.499 94) (end 158.873 94.5399) (width 0.8002) (layer F.Cu) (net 5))
 (segment (start 158.499 94) (end 158.05 94.4799) (width 0.8002) (layer F.Cu) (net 5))
 (segment (start 158.499 94) (end 158.438 94.8417) (width 0.8002) (layer F.Cu) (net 5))
 (segment (start 158.438 94.8417) (end 157.888 99.3318) (width 1.86) (layer F.Cu) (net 5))
 (segment (start 157.888 99.3318) (end 157.522 102.826) (width 1.86) (layer F.Cu) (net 5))
 (segment (start 157.888 99.3318) (end 131.5 102) (width 1.86) (layer F.Cu) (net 5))
 (segment (start 172.6355 100.671) (end 172.429 100.671) (width 0.25) (layer F.Cu) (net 7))
 (segment (start 172.429 100.671) (end 172.1 101) (width 0.25) (layer F.Cu) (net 7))
 (segment (start 172.6355 100.671) (end 172.211 100.978) (width 0.9) (layer F.Cu) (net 7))
 (segment (start 172.211 100.978) (end 173.23 101.22) (width 0.9) (layer F.Cu) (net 7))
 (segment (start 173.06 100.364) (end 172.6355 100.671) (width 0.9) (layer F.Cu) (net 7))
 (segment (start 172.1 101) (end 173.341 100.753) (width 0.9) (layer F.Cu) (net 7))
 (segment (start 176.5 99) (end 175.197 99.8343) (width 1.86) (layer F.Cu) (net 7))
 (segment (start 175.197 99.8343) (end 173.341 100.753) (width 1.86) (layer F.Cu) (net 7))
 (segment (start 161.7598 111.3034) (end 161.297 110.488) (width 0.9) (layer F.Cu) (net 8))
 (segment (start 160.787 111.196) (end 161.814 111.399) (width 0.9) (layer F.Cu) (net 8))
 (segment (start 161.814 111.399) (end 161.7598 111.3034) (width 0.9) (layer F.Cu) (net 8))
 (segment (start 161.7158 111.3284) (end 161.7348 111.3284) (width 0.25) (layer F.Cu) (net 8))
 (segment (start 161.7348 111.3284) (end 161.7598 111.3034) (width 0.25) (layer F.Cu) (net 8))
 (segment (start 161.7158 111.3284) (end 160.88 110.725) (width 0.9) (layer F.Cu) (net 8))
 (segment (start 162.146 111.639) (end 161.7158 111.3284) (width 0.9) (layer F.Cu) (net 8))
 (segment (start 161.3208 104.694) (end 161.5 104.1) (width 0.9) (layer F.Cu) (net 8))
 (segment (start 161.084 105.479) (end 161.3208 104.694) (width 0.9) (layer F.Cu) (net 8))
 (segment (start 161.4666 104.738) (end 161.3648 104.738) (width 0.25) (layer F.Cu) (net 8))
 (segment (start 161.3648 104.738) (end 161.3208 104.694) (width 0.25) (layer F.Cu) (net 8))
 (segment (start 161.559 105.413) (end 161.4666 104.738) (width 0.9) (layer F.Cu) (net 8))
 (segment (start 161.4666 104.738) (end 161.417 104.376) (width 0.9) (layer F.Cu) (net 8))
 (segment (start 161.417 104.376) (end 160.724 105.161) (width 0.9) (layer F.Cu) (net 8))
 (segment (start 157.5 106.6) (end 158.2751 106.6) (width 0.25) (layer F.Cu) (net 8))
 (segment (start 158.3295 106.473) (end 158.2751 106.5274) (width 0.25) (layer F.Cu) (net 8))
 (segment (start 158.2751 106.5274) (end 158.2751 106.6) (width 0.25) (layer F.Cu) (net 8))
 (segment (start 158.3295 106.473) (end 157.832 106.637) (width 0.9) (layer F.Cu) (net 8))
 (segment (start 157.832 106.637) (end 158.73 107.176) (width 0.9) (layer F.Cu) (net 8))
 (segment (start 158.827 106.309) (end 158.3295 106.473) (width 0.9) (layer F.Cu) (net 8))
 (segment (start 157.5 106.6) (end 158.977 106.765) (width 0.9) (layer F.Cu) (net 8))
 (segment (start 158.977 106.765) (end 161.084 105.479) (width 1.86) (layer F.Cu) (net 8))
 (segment (start 160.88 110.725) (end 158.977 106.765) (width 1.86) (layer F.Cu) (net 8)))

